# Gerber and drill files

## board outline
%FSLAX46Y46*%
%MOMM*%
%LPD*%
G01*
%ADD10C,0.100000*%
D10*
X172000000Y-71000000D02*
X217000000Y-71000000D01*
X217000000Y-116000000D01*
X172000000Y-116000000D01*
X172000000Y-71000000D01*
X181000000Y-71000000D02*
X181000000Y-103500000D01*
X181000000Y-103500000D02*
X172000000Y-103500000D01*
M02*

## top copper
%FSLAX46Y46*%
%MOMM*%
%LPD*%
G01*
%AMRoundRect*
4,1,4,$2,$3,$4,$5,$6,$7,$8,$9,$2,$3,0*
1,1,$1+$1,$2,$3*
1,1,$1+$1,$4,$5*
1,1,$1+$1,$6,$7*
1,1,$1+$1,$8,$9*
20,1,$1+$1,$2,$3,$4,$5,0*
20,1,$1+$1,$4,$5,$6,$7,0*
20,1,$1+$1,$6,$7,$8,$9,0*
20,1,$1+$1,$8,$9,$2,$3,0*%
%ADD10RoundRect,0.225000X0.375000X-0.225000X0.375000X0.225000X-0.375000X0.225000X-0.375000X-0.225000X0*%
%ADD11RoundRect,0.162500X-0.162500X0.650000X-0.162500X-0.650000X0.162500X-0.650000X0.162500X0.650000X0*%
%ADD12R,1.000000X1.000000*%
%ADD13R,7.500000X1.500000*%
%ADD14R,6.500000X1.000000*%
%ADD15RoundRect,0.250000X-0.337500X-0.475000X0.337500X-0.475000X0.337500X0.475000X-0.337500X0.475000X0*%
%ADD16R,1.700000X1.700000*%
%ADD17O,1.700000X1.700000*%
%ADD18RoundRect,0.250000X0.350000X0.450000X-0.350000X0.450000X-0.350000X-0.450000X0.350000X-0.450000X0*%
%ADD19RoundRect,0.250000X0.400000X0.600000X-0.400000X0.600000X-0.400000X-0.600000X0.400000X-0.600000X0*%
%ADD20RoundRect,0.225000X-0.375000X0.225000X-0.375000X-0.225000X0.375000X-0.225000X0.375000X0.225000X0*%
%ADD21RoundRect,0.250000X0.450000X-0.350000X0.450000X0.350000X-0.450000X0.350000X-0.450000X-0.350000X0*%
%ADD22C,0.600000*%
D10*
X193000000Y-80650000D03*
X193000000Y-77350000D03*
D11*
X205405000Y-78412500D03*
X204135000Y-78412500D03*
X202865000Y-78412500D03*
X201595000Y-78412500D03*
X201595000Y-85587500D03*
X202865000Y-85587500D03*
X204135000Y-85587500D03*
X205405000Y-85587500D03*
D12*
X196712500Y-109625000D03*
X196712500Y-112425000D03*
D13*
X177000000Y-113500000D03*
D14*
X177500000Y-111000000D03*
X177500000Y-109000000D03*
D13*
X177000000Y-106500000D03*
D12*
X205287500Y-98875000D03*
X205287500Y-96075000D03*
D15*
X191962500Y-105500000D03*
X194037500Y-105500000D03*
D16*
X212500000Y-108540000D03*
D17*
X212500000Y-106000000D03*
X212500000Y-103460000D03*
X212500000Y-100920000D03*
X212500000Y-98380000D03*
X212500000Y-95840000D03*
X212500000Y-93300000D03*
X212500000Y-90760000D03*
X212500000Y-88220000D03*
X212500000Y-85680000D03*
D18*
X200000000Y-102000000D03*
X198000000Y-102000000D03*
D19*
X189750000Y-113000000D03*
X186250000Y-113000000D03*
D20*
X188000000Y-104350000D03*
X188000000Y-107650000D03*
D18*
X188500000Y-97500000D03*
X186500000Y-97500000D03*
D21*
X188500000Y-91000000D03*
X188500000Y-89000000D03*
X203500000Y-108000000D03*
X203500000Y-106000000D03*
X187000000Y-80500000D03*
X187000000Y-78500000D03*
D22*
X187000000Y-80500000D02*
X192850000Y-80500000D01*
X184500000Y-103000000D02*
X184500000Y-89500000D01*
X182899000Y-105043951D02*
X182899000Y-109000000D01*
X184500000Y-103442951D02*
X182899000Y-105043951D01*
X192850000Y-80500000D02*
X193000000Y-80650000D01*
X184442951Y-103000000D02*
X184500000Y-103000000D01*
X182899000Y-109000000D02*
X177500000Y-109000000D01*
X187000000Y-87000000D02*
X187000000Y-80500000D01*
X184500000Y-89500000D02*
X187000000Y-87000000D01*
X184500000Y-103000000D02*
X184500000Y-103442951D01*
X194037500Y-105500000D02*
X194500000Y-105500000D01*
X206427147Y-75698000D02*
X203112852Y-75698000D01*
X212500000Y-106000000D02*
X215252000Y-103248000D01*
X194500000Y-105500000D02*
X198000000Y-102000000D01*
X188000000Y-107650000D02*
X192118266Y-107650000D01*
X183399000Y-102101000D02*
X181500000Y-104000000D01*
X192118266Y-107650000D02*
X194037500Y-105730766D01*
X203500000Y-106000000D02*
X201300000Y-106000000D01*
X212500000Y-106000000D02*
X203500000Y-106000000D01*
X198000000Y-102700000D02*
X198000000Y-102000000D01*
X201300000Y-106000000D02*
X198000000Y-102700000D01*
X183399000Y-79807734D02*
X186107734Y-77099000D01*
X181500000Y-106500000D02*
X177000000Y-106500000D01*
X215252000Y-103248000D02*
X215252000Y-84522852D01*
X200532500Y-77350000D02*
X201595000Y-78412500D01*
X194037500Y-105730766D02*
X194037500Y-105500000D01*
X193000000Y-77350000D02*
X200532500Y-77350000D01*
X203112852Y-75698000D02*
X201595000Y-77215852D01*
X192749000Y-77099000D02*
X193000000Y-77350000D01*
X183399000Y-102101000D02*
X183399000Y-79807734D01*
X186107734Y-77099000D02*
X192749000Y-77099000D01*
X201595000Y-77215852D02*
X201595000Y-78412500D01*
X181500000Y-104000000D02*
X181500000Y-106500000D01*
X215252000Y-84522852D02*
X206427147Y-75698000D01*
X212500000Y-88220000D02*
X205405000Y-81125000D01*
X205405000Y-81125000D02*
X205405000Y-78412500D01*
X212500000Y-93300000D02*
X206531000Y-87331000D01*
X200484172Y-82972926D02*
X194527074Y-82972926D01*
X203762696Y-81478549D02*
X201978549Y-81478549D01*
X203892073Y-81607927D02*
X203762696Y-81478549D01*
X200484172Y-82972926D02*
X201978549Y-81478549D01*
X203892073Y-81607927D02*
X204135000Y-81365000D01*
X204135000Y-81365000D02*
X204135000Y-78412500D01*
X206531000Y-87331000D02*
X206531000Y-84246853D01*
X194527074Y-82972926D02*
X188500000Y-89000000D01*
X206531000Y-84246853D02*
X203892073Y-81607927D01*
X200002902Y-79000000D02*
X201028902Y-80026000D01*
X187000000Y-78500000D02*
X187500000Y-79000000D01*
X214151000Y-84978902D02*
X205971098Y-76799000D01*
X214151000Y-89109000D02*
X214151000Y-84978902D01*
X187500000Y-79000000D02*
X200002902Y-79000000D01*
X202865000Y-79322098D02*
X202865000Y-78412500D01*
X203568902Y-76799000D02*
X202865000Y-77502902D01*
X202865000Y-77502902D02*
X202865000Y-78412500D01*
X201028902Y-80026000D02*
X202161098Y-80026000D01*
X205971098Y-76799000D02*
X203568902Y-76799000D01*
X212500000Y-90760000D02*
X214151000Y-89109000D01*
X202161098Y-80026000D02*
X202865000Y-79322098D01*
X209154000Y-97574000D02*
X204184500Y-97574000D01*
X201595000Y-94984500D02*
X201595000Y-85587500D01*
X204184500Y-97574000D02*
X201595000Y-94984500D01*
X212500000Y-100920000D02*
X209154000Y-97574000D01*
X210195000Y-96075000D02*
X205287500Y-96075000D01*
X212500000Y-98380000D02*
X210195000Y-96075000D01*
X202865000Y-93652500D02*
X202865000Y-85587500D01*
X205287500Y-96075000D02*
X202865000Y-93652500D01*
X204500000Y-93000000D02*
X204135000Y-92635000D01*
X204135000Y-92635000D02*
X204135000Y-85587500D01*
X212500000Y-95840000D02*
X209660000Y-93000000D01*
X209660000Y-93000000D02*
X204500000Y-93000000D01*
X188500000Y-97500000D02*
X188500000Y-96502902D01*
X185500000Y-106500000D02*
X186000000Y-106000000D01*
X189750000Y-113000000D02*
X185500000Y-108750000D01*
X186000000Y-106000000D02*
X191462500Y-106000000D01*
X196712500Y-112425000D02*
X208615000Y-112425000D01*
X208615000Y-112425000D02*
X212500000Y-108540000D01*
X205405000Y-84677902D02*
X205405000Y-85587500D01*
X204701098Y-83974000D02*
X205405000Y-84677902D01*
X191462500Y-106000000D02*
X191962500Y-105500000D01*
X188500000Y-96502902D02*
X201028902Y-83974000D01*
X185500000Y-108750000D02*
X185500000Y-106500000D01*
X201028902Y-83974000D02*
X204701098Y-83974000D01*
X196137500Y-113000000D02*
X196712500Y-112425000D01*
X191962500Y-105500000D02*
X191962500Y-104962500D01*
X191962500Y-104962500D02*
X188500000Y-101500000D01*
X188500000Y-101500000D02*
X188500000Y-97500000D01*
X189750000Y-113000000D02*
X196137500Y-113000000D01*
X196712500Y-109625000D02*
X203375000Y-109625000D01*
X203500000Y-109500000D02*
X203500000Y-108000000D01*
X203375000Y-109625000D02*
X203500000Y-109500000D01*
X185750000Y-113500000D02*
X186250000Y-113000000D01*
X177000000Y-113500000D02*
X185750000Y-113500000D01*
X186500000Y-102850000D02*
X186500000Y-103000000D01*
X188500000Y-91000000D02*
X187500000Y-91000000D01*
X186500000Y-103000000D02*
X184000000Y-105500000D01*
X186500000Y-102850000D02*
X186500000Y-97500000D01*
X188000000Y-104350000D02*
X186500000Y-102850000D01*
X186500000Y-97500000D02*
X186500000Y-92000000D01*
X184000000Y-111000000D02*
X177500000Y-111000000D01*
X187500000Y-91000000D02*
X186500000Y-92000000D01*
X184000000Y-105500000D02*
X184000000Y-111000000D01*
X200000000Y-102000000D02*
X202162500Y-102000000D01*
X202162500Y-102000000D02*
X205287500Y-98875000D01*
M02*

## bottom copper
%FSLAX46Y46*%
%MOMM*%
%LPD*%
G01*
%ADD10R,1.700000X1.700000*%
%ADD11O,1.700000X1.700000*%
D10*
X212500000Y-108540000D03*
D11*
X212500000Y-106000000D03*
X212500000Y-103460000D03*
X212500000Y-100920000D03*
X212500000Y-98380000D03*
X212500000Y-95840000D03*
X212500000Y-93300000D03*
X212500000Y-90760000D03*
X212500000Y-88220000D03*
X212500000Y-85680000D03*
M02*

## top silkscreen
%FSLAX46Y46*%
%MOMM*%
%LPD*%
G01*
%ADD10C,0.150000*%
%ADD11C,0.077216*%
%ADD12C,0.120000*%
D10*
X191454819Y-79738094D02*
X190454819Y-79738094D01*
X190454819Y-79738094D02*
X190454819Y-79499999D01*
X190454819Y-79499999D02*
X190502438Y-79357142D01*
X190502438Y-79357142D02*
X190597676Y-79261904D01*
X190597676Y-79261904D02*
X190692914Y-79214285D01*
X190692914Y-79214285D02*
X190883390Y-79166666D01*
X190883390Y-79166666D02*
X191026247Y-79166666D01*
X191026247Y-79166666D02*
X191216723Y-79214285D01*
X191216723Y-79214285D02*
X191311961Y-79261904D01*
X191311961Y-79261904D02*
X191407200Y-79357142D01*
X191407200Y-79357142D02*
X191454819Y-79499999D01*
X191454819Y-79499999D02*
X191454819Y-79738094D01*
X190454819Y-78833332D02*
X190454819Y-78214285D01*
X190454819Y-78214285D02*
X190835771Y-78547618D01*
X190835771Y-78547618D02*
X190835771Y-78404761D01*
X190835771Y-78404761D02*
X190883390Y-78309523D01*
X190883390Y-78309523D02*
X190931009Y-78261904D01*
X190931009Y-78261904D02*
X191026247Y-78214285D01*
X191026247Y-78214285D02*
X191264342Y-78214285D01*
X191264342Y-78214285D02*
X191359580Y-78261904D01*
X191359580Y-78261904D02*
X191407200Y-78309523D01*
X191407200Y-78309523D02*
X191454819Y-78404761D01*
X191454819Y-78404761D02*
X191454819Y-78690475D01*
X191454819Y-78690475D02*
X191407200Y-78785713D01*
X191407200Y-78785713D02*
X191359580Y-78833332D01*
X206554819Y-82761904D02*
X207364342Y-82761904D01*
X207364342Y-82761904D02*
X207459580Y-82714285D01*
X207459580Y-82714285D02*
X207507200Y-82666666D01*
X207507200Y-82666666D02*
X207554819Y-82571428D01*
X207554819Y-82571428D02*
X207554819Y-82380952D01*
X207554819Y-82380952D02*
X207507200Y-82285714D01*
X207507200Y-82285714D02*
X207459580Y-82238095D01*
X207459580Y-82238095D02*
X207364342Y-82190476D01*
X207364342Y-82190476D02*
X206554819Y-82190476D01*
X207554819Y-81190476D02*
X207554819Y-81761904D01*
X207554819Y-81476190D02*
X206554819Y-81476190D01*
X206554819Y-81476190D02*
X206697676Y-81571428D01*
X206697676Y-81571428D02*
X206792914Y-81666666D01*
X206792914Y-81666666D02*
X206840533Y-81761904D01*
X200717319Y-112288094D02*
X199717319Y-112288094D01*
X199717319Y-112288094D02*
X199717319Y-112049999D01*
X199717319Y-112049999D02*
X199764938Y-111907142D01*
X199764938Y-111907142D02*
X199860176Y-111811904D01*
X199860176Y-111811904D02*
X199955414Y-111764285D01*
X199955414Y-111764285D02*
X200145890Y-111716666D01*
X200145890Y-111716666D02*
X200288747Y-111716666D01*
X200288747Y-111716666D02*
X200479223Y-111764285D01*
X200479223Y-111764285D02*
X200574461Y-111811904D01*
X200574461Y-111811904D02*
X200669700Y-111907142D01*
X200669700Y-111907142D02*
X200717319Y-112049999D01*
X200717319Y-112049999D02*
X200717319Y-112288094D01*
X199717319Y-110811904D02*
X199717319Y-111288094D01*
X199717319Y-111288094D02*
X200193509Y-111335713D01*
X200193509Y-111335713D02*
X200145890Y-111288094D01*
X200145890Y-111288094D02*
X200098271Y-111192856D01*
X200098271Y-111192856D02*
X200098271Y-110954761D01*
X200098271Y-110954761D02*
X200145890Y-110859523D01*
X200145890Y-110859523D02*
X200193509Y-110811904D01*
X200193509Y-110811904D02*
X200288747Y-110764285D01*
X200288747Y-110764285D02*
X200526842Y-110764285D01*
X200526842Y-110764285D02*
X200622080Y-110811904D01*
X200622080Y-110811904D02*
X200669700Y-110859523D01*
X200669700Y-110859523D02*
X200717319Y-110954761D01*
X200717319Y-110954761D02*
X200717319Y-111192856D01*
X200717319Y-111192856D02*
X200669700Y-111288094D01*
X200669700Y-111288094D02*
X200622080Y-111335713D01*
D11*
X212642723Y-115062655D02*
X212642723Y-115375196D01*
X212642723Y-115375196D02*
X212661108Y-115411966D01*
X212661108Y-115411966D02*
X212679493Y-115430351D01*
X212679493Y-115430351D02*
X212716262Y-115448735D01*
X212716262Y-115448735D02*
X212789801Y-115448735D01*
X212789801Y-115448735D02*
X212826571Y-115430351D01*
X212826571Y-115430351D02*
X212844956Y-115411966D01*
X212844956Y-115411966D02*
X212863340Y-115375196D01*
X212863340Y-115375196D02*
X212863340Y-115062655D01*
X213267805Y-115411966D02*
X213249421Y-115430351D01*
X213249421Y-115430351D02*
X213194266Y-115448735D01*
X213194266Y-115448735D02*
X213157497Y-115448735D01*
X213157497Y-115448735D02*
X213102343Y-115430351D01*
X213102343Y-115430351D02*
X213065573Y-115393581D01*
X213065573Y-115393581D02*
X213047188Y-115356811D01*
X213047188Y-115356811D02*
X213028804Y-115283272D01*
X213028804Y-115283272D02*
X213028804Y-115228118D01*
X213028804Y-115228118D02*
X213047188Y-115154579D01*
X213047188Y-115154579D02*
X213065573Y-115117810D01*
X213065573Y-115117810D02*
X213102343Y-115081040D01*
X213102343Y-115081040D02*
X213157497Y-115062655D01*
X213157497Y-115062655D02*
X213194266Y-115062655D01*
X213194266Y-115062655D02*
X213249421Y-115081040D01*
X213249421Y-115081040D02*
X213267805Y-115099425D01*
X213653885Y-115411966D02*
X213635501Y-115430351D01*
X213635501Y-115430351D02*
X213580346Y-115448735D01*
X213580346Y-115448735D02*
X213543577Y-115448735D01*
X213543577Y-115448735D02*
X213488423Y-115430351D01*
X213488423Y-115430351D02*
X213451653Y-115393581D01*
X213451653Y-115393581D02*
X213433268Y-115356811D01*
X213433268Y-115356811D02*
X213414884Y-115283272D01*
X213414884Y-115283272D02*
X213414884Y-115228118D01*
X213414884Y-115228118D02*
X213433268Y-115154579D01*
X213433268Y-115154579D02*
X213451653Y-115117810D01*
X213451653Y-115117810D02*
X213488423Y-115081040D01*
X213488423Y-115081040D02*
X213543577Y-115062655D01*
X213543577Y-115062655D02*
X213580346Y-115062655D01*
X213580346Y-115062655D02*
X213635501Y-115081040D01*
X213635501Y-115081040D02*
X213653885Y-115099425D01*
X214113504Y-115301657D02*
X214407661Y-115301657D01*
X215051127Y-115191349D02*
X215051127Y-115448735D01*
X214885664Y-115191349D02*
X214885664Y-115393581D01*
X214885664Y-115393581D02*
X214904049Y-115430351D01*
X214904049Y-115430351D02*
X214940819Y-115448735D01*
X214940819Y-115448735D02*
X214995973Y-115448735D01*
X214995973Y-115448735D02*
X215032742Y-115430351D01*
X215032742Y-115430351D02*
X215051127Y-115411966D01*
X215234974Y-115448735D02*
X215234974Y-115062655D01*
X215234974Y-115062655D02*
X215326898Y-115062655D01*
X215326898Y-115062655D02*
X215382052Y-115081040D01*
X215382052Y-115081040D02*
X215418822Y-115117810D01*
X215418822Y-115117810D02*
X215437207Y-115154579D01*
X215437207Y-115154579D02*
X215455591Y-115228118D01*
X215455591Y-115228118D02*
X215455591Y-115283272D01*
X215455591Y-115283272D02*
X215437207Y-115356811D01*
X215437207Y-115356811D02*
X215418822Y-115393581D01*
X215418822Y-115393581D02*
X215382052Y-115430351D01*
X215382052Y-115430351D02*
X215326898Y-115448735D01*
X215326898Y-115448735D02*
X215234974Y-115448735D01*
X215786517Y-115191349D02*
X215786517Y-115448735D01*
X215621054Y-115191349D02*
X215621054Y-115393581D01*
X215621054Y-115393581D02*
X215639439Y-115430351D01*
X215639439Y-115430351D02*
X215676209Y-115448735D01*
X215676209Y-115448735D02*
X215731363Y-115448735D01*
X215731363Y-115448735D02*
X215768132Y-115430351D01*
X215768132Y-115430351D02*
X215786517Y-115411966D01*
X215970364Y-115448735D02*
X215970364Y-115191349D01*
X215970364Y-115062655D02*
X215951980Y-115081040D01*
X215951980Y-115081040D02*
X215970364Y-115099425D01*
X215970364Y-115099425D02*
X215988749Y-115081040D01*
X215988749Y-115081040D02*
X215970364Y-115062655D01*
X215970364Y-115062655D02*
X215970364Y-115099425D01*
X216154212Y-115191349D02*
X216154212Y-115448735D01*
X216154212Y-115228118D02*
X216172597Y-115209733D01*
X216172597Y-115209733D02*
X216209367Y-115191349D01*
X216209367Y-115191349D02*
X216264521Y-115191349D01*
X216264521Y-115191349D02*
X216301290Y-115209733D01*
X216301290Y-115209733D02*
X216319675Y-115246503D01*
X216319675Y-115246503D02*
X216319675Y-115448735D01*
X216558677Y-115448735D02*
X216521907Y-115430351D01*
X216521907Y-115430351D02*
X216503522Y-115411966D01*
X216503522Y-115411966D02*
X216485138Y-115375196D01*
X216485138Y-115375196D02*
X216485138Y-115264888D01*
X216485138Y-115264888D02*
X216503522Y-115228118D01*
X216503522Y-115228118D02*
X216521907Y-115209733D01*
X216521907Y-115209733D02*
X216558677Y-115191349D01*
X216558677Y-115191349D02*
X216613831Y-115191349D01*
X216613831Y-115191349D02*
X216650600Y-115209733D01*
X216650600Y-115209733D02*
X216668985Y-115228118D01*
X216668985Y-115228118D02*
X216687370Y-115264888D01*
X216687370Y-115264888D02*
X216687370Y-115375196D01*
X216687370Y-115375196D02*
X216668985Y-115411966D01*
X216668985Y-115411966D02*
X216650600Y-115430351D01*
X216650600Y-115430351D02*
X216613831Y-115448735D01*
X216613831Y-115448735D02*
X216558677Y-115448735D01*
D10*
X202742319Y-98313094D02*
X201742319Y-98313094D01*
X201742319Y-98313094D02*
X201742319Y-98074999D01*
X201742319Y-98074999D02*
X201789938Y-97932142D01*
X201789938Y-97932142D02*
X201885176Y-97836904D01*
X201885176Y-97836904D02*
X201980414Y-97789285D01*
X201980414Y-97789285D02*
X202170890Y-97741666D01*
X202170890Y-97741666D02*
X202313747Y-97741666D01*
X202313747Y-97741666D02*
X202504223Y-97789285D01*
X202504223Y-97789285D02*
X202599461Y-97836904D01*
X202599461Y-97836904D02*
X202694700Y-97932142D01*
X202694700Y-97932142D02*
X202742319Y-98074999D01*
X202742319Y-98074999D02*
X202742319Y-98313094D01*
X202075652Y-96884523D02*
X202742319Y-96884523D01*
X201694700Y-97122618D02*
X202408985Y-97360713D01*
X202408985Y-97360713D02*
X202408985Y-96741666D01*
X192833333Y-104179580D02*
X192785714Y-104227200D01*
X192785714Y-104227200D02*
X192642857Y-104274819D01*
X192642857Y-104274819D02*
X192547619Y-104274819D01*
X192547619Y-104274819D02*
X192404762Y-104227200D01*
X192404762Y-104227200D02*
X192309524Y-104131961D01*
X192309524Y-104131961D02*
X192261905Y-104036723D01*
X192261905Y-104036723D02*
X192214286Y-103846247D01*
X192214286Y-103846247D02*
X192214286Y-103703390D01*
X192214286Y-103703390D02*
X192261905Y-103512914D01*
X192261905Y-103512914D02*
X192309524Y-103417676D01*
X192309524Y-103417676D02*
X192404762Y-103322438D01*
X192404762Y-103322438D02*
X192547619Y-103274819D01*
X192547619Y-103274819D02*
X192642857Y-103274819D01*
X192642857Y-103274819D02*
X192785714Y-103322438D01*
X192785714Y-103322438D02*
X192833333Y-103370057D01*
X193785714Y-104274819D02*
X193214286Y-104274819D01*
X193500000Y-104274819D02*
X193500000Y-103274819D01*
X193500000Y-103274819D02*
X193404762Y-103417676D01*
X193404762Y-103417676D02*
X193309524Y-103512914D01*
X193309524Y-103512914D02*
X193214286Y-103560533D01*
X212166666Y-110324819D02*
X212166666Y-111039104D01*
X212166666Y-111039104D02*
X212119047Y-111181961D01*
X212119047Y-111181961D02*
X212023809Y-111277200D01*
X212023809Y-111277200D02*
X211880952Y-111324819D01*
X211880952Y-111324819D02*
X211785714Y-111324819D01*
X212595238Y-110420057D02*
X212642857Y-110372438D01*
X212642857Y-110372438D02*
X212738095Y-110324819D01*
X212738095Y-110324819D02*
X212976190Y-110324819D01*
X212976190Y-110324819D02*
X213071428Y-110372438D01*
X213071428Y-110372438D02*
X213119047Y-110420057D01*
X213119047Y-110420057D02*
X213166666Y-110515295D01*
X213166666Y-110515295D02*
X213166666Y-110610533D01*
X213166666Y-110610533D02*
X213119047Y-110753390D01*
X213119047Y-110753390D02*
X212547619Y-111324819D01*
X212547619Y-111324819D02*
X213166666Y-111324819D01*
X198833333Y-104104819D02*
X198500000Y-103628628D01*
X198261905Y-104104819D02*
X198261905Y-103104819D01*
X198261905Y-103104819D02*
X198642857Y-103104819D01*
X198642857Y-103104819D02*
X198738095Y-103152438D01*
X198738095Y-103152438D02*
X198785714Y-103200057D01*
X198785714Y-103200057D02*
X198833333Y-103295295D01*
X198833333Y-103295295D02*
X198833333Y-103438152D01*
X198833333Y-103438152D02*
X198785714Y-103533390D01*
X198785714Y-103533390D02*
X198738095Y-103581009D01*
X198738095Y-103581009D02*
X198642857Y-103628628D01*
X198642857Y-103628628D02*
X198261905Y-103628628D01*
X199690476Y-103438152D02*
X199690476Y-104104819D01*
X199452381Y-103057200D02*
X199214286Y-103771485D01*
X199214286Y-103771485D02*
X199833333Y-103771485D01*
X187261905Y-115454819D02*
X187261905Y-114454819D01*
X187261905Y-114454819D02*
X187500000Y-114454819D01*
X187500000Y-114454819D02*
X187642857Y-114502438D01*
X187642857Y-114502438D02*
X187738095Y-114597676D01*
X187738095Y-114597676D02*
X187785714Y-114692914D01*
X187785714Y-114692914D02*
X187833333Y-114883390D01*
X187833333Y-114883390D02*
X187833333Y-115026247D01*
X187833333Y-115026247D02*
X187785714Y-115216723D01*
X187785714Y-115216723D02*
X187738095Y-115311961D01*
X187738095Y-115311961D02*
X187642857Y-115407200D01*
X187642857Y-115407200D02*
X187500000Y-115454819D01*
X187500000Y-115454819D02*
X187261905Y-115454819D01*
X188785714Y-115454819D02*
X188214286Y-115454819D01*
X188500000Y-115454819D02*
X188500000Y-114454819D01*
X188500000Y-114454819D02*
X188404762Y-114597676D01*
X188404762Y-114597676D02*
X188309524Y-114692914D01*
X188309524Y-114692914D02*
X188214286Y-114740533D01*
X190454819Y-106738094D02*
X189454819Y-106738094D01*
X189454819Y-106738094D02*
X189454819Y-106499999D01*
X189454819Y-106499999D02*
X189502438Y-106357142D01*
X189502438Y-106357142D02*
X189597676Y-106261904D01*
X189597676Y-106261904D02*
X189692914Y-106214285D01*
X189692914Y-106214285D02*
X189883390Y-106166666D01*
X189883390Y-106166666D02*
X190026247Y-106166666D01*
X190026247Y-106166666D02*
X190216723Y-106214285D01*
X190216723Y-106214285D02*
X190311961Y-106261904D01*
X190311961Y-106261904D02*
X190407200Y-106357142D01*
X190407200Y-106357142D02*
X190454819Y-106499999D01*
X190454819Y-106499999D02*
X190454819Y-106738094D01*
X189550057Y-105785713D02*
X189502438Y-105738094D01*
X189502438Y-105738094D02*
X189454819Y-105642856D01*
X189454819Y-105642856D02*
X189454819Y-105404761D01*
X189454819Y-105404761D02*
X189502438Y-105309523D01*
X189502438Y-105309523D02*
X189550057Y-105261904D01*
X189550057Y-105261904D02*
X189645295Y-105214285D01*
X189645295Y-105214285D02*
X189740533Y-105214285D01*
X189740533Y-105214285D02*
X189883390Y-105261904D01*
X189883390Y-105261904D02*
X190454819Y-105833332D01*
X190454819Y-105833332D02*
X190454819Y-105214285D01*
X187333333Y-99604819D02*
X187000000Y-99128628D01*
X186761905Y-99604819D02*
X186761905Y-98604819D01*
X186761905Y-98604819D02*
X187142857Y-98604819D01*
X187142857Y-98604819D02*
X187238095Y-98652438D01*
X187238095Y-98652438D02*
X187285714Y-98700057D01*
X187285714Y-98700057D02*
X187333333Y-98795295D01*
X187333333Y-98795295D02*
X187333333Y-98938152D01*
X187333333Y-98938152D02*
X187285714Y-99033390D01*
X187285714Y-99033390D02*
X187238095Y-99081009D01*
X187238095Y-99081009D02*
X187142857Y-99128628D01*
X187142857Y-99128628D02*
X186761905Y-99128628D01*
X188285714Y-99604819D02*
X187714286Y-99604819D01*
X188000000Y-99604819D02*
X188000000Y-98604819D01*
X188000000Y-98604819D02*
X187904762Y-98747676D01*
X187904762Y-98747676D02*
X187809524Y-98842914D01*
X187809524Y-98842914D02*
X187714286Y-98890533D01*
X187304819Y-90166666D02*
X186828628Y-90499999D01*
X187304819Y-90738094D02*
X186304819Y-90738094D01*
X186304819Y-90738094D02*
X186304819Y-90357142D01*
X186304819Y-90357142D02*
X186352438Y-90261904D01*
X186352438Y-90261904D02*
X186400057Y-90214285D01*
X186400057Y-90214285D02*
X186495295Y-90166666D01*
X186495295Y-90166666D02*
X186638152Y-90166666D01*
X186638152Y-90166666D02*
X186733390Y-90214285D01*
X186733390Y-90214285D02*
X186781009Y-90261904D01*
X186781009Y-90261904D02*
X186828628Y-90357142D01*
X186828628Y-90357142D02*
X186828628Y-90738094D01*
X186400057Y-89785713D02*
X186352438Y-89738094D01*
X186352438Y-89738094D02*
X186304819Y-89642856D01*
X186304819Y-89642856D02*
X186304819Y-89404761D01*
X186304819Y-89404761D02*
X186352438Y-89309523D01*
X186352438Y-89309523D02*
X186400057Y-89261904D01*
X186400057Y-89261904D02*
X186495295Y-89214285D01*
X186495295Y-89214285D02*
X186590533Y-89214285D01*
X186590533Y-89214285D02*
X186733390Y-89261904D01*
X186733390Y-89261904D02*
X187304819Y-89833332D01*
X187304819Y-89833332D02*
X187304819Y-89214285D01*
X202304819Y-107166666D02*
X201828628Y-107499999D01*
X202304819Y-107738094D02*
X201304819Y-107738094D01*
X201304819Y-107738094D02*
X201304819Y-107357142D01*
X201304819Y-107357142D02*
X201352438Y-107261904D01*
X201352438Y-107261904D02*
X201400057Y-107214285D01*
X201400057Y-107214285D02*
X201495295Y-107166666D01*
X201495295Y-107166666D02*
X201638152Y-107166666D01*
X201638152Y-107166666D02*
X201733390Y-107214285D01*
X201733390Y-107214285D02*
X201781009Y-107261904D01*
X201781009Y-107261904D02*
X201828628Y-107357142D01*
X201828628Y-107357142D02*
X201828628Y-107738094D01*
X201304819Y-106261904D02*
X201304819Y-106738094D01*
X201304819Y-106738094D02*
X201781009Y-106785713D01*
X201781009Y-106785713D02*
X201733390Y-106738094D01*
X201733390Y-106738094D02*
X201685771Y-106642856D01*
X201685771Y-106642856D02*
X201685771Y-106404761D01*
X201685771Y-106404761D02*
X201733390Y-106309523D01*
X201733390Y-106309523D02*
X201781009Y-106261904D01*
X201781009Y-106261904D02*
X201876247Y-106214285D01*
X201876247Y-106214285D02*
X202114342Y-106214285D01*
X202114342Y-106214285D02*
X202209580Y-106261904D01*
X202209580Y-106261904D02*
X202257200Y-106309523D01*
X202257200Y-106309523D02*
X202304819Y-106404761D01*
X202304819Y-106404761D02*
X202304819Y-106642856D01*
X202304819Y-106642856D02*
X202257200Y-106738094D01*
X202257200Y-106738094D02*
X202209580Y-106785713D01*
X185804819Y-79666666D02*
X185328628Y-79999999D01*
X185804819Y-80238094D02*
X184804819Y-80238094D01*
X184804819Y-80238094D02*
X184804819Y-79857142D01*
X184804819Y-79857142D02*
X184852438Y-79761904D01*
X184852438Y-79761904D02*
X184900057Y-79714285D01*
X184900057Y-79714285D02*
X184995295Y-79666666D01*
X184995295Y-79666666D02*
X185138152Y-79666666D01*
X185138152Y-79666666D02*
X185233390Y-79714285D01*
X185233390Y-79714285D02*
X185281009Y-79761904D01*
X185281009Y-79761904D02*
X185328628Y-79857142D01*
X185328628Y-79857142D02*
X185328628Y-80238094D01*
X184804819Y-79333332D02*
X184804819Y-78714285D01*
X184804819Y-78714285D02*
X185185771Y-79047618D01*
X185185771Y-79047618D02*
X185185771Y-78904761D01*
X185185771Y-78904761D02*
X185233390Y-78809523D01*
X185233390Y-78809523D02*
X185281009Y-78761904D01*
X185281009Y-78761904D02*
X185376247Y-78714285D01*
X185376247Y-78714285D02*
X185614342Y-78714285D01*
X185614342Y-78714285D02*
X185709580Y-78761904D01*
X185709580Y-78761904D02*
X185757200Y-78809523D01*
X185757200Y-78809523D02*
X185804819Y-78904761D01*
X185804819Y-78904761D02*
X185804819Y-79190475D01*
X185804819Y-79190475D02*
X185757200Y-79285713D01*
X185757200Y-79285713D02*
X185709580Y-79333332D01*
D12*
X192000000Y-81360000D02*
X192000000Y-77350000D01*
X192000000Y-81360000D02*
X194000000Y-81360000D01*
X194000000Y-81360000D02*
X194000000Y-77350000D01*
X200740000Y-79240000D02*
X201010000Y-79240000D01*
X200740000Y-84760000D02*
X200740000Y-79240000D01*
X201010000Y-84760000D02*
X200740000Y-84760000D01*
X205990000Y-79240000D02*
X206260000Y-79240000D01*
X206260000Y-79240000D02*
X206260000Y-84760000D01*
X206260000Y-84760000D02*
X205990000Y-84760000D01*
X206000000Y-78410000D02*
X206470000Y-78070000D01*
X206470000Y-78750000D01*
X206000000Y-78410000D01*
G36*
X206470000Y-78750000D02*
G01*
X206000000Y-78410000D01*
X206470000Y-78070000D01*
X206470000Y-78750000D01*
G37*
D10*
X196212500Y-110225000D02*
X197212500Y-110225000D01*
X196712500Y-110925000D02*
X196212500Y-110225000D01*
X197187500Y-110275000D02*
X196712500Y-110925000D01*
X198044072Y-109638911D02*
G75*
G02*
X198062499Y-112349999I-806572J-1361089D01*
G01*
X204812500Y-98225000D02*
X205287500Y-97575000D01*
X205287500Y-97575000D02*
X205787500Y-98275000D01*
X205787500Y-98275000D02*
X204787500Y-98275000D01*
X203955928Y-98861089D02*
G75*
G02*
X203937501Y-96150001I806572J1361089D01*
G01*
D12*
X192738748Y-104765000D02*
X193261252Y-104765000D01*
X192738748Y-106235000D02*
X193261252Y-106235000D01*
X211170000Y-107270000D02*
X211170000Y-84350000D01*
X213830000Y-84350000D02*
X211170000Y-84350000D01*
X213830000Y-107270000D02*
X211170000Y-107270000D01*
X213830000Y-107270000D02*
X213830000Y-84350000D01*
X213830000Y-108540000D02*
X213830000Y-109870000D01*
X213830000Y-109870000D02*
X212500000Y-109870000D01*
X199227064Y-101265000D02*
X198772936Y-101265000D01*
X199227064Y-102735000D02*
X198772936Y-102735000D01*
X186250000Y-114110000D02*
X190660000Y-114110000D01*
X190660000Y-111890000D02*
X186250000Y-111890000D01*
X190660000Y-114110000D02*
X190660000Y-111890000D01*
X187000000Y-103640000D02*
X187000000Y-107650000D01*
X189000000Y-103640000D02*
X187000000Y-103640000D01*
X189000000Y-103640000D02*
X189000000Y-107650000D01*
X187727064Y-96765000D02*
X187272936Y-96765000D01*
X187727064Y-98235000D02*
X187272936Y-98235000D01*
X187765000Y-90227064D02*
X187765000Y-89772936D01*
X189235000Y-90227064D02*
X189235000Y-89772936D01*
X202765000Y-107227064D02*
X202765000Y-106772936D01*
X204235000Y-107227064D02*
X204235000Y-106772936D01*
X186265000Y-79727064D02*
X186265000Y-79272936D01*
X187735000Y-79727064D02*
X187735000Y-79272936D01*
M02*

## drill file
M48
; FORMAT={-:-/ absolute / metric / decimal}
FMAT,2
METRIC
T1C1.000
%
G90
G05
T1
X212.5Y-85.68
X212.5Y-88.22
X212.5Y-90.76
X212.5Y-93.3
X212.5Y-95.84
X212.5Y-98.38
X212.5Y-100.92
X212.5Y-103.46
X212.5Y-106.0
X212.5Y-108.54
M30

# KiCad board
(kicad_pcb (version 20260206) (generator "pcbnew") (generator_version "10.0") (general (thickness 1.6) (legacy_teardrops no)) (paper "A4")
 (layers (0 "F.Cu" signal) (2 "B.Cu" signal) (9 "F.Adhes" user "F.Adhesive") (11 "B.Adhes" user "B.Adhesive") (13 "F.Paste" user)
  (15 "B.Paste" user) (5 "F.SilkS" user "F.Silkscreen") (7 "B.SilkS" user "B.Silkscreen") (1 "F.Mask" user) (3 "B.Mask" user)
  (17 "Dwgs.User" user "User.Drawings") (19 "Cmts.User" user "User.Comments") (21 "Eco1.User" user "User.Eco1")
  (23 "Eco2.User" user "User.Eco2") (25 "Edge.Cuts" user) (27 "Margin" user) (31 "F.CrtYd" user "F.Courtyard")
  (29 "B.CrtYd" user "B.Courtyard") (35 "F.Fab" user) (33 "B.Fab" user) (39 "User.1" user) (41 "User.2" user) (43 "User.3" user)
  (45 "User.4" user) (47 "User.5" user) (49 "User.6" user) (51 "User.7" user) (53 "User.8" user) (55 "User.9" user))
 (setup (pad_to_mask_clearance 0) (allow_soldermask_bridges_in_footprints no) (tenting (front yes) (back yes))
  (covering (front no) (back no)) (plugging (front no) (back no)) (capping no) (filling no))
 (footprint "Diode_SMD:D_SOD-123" (layer "F.Cu") (at 193 79 90)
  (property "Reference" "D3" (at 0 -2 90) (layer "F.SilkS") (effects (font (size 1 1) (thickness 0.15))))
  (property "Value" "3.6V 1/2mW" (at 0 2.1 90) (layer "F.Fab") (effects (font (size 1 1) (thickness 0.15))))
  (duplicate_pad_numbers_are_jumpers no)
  (fp_line (start -2.36 -1) (end 1.65 -1) (stroke (width 0.12) (type solid)) (layer "F.SilkS"))
  (fp_line (start -2.36 -1) (end -2.36 1) (stroke (width 0.12) (type solid)) (layer "F.SilkS"))
  (fp_line (start -2.36 1) (end 1.65 1) (stroke (width 0.12) (type solid)) (layer "F.SilkS"))
  (pad "1" smd roundrect (at -1.65 0 90) (size 0.9 1.2) (layers "F.Cu" "F.Mask" "F.Paste") (roundrect_rratio 0.25) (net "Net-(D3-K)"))
  (pad "2" smd roundrect (at 1.65 0 90) (size 0.9 1.2) (layers "F.Cu" "F.Mask" "F.Paste") (roundrect_rratio 0.25) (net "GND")))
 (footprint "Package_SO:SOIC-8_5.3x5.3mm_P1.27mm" (layer "F.Cu") (at 203.5 82 -90)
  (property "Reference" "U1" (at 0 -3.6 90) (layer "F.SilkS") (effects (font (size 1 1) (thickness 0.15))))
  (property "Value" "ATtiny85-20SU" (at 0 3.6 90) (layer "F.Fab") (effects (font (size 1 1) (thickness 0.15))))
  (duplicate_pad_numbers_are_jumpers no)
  (fp_line (start -2.76 2.76) (end -2.76 2.49) (stroke (width 0.12) (type solid)) (layer "F.SilkS"))
  (fp_line (start 2.76 2.76) (end -2.76 2.76) (stroke (width 0.12) (type solid)) (layer "F.SilkS"))
  (fp_line (start 2.76 2.49) (end 2.76 2.76) (stroke (width 0.12) (type solid)) (layer "F.SilkS"))
  (fp_line (start -2.76 -2.49) (end -2.76 -2.76) (stroke (width 0.12) (type solid)) (layer "F.SilkS"))
  (fp_line (start -2.76 -2.76) (end 2.76 -2.76) (stroke (width 0.12) (type solid)) (layer "F.SilkS"))
  (fp_line (start 2.76 -2.76) (end 2.76 -2.49) (stroke (width 0.12) (type solid)) (layer "F.SilkS"))
  (fp_poly (pts (xy -3.59 -2.5) (xy -3.93 -2.97) (xy -3.25 -2.97)) (stroke (width 0.12) (type solid)) (fill yes) (layer "F.SilkS"))
  (pad "1" smd roundrect (at -3.5875 -1.905 270) (size 1.625 0.65) (layers "F.Cu" "F.Mask" "F.Paste") (roundrect_rratio 0.25)
   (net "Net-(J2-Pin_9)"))
  (pad "2" smd roundrect (at -3.5875 -0.635 270) (size 1.625 0.65) (layers "F.Cu" "F.Mask" "F.Paste") (roundrect_rratio 0.25)
   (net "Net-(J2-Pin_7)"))
  (pad "3" smd roundrect (at -3.5875 0.635 270) (size 1.625 0.65) (layers "F.Cu" "F.Mask" "F.Paste") (roundrect_rratio 0.25)
   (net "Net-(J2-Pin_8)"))
  (pad "4" smd roundrect (at -3.5875 1.905 270) (size 1.625 0.65) (layers "F.Cu" "F.Mask" "F.Paste") (roundrect_rratio 0.25) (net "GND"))
  (pad "5" smd roundrect (at 3.5875 1.905 270) (size 1.625 0.65) (layers "F.Cu" "F.Mask" "F.Paste") (roundrect_rratio 0.25)
   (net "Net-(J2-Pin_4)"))
  (pad "6" smd roundrect (at 3.5875 0.635 270) (size 1.625 0.65) (layers "F.Cu" "F.Mask" "F.Paste") (roundrect_rratio 0.25)
   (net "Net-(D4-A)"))
  (pad "7" smd roundrect (at 3.5875 -0.635 270) (size 1.625 0.65) (layers "F.Cu" "F.Mask" "F.Paste") (roundrect_rratio 0.25)
   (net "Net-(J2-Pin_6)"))
  (pad "8" smd roundrect (at 3.5875 -1.905 270) (size 1.625 0.65) (layers "F.Cu" "F.Mask" "F.Paste") (roundrect_rratio 0.25) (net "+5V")))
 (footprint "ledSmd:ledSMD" (layer "F.Cu") (at 196.7125 111.425 -90)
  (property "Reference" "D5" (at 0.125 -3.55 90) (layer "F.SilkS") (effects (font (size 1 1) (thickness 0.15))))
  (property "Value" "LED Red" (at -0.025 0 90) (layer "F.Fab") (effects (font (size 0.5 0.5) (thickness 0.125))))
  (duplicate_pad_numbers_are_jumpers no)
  (fp_line (start -1.2 0.5) (end -1.2 -0.5) (stroke (width 0.15) (type solid)) (layer "F.SilkS"))
  (fp_line (start -0.5 0) (end -1.2 0.5) (stroke (width 0.15) (type solid)) (layer "F.SilkS"))
  (fp_line (start -1.15 -0.475) (end -0.5 0) (stroke (width 0.15) (type solid)) (layer "F.SilkS"))
  (fp_arc (start -1.786089 -1.331572) (mid -0.435753 -2.107089) (end 0.924999 -1.349999) (stroke (width 0.15) (type solid))
   (layer "F.SilkS"))
  (pad "1" smd rect (at -1.8 0 270) (size 1 1) (layers "F.Cu" "F.Mask" "F.Paste") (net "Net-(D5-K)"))
  (pad "2" smd rect (at 1 0 270) (size 1 1) (layers "F.Cu" "F.Mask" "F.Paste") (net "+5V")))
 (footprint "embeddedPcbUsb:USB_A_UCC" (layer "F.Cu") (at 177.2 110)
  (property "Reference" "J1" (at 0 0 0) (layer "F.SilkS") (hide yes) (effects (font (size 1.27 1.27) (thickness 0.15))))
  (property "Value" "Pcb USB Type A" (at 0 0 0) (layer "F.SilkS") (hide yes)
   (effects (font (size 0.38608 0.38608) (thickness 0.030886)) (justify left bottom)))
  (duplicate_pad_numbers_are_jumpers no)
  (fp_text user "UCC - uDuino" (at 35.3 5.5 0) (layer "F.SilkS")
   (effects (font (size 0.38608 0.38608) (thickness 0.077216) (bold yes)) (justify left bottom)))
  (pad "1" smd rect (at -0.2 3.5) (size 7.5 1.5) (layers "F.Cu" "F.Mask" "F.Paste") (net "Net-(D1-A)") (solder_mask_margin 0.1016))
  (pad "2" smd rect (at 0.3 1) (size 6.5 1) (layers "F.Cu" "F.Mask" "F.Paste") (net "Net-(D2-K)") (solder_mask_margin 0.1016))
  (pad "3" smd rect (at 0.3 -1) (size 6.5 1) (layers "F.Cu" "F.Mask" "F.Paste") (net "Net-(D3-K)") (solder_mask_margin 0.1016))
  (pad "4" smd rect (at -0.2 -3.5) (size 7.5 1.5) (layers "F.Cu" "F.Mask" "F.Paste") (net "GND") (solder_mask_margin 0.1016)))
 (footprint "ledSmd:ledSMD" (layer "F.Cu") (at 205.2875 97.075 90)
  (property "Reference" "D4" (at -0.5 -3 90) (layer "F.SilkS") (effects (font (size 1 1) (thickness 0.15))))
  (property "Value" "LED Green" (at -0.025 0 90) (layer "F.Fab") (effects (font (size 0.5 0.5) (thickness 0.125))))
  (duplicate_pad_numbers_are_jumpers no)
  (fp_line (start -1.15 -0.475) (end -0.5 0) (stroke (width 0.15) (type solid)) (layer "F.SilkS"))
  (fp_line (start -0.5 0) (end -1.2 0.5) (stroke (width 0.15) (type solid)) (layer "F.SilkS"))
  (fp_line (start -1.2 0.5) (end -1.2 -0.5) (stroke (width 0.15) (type solid)) (layer "F.SilkS"))
  (fp_arc (start -1.786089 -1.331572) (mid -0.435753 -2.107089) (end 0.924999 -1.349999) (stroke (width 0.15) (type solid))
   (layer "F.SilkS"))
  (pad "1" smd rect (at -1.8 0 90) (size 1 1) (layers "F.Cu" "F.Mask" "F.Paste") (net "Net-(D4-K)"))
  (pad "2" smd rect (at 1 0 90) (size 1 1) (layers "F.Cu" "F.Mask" "F.Paste") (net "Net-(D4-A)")))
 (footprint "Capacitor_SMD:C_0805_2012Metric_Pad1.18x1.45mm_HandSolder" (layer "F.Cu") (at 193 105.5)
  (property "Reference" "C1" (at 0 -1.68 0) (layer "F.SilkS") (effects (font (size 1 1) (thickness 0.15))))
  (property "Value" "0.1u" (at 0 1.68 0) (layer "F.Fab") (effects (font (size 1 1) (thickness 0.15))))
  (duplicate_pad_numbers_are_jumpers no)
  (fp_line (start -0.261252 -0.735) (end 0.261252 -0.735) (stroke (width 0.12) (type solid)) (layer "F.SilkS"))
  (fp_line (start -0.261252 0.735) (end 0.261252 0.735) (stroke (width 0.12) (type solid)) (layer "F.SilkS"))
  (pad "1" smd roundrect (at -1.0375 0) (size 1.175 1.45) (layers "F.Cu" "F.Mask" "F.Paste") (roundrect_rratio 0.212766) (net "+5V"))
  (pad "2" smd roundrect (at 1.0375 0) (size 1.175 1.45) (layers "F.Cu" "F.Mask" "F.Paste") (roundrect_rratio 0.212766) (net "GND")))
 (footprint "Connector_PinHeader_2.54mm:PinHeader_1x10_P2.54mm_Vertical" (layer "F.Cu") (at 212.5 108.54 180)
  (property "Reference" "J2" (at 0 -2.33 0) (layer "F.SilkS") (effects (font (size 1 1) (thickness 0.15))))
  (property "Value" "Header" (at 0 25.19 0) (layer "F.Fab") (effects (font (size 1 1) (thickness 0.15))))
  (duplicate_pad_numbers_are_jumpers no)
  (fp_line (start 1.33 1.27) (end 1.33 24.19) (stroke (width 0.12) (type solid)) (layer "F.SilkS"))
  (fp_line (start -1.33 24.19) (end 1.33 24.19) (stroke (width 0.12) (type solid)) (layer "F.SilkS"))
  (fp_line (start -1.33 1.27) (end 1.33 1.27) (stroke (width 0.12) (type solid)) (layer "F.SilkS"))
  (fp_line (start -1.33 1.27) (end -1.33 24.19) (stroke (width 0.12) (type solid)) (layer "F.SilkS"))
  (fp_line (start -1.33 0) (end -1.33 -1.33) (stroke (width 0.12) (type solid)) (layer "F.SilkS"))
  (fp_line (start -1.33 -1.33) (end 0 -1.33) (stroke (width 0.12) (type solid)) (layer "F.SilkS"))
  (pad "1" thru_hole rect (at 0 0 180) (size 1.7 1.7) (drill 1) (layers "*.Cu" "*.Mask") (remove_unused_layers no) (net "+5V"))
  (pad "2" thru_hole oval (at 0 2.54 180) (size 1.7 1.7) (drill 1) (layers "*.Cu" "*.Mask") (remove_unused_layers no) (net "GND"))
  (pad "3" thru_hole oval (at 0 5.08 180) (size 1.7 1.7) (drill 1) (layers "*.Cu" "*.Mask") (remove_unused_layers no)
   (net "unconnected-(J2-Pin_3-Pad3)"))
  (pad "4" thru_hole oval (at 0 7.62 180) (size 1.7 1.7) (drill 1) (layers "*.Cu" "*.Mask") (remove_unused_layers no) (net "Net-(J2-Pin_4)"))
  (pad "5" thru_hole oval (at 0 10.16 180) (size 1.7 1.7) (drill 1) (layers "*.Cu" "*.Mask") (remove_unused_layers no) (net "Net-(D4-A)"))
  (pad "6" thru_hole oval (at 0 12.7 180) (size 1.7 1.7) (drill 1) (layers "*.Cu" "*.Mask") (remove_unused_layers no) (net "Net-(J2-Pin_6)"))
  (pad "7" thru_hole oval (at 0 15.24 180) (size 1.7 1.7) (drill 1) (layers "*.Cu" "*.Mask") (remove_unused_layers no)
   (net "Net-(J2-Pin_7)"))
  (pad "8" thru_hole oval (at 0 17.78 180) (size 1.7 1.7) (drill 1) (layers "*.Cu" "*.Mask") (remove_unused_layers no)
   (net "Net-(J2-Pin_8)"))
  (pad "9" thru_hole oval (at 0 20.32 180) (size 1.7 1.7) (drill 1) (layers "*.Cu" "*.Mask") (remove_unused_layers no)
   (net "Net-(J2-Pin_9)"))
  (pad "10" thru_hole oval (at 0 22.86 180) (size 1.7 1.7) (drill 1) (layers "*.Cu" "*.Mask") (remove_unused_layers no)
   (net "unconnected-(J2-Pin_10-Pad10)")))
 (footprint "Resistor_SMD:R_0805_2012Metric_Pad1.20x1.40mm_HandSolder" (layer "F.Cu") (at 199 102 180)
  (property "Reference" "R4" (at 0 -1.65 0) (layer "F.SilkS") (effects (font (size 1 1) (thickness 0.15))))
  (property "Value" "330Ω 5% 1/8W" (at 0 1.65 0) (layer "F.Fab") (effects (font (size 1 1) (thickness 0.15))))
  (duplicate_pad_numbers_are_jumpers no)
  (fp_line (start -0.227064 0.735) (end 0.227064 0.735) (stroke (width 0.12) (type solid)) (layer "F.SilkS"))
  (fp_line (start -0.227064 -0.735) (end 0.227064 -0.735) (stroke (width 0.12) (type solid)) (layer "F.SilkS"))
  (pad "1" smd roundrect (at -1 0 180) (size 1.2 1.4) (layers "F.Cu" "F.Mask" "F.Paste") (roundrect_rratio 0.208333) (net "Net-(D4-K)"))
  (pad "2" smd roundrect (at 1 0 180) (size 1.2 1.4) (layers "F.Cu" "F.Mask" "F.Paste") (roundrect_rratio 0.208333) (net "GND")))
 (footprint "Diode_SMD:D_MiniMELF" (layer "F.Cu") (at 188 113 180)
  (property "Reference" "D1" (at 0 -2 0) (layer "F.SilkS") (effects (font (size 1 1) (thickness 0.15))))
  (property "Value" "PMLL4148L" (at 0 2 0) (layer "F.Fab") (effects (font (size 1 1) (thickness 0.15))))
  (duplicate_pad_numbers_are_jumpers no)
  (fp_line (start 1.75 -1.11) (end -2.66 -1.11) (stroke (width 0.12) (type solid)) (layer "F.SilkS"))
  (fp_line (start -2.66 1.11) (end 1.75 1.11) (stroke (width 0.12) (type solid)) (layer "F.SilkS"))
  (fp_line (start -2.66 -1.11) (end -2.66 1.11) (stroke (width 0.12) (type solid)) (layer "F.SilkS"))
  (pad "1" smd roundrect (at -1.75 0 180) (size 1.3 1.7) (layers "F.Cu" "F.Mask" "F.Paste") (roundrect_rratio 0.1923076923) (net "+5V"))
  (pad "2" smd roundrect (at 1.75 0 180) (size 1.3 1.7) (layers "F.Cu" "F.Mask" "F.Paste") (roundrect_rratio 0.1923076923)
   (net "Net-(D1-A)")))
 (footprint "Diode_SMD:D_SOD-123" (layer "F.Cu") (at 188 106 -90)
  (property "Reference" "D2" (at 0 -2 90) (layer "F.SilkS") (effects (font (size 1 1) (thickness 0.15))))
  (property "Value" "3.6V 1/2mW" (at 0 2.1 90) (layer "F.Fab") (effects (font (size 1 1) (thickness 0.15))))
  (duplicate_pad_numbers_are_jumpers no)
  (fp_line (start -2.36 1) (end 1.65 1) (stroke (width 0.12) (type solid)) (layer "F.SilkS"))
  (fp_line (start -2.36 -1) (end -2.36 1) (stroke (width 0.12) (type solid)) (layer "F.SilkS"))
  (fp_line (start -2.36 -1) (end 1.65 -1) (stroke (width 0.12) (type solid)) (layer "F.SilkS"))
  (pad "1" smd roundrect (at -1.65 0 270) (size 0.9 1.2) (layers "F.Cu" "F.Mask" "F.Paste") (roundrect_rratio 0.25) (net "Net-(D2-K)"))
  (pad "2" smd roundrect (at 1.65 0 270) (size 0.9 1.2) (layers "F.Cu" "F.Mask" "F.Paste") (roundrect_rratio 0.25) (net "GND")))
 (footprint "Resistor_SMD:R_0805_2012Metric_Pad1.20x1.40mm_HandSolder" (layer "F.Cu") (at 187.5 97.5 180)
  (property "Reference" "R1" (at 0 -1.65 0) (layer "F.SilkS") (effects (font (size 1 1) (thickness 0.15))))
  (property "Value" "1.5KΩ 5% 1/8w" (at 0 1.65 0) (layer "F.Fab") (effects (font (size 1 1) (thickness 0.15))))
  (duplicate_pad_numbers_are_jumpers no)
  (fp_line (start -0.227064 0.735) (end 0.227064 0.735) (stroke (width 0.12) (type solid)) (layer "F.SilkS"))
  (fp_line (start -0.227064 -0.735) (end 0.227064 -0.735) (stroke (width 0.12) (type solid)) (layer "F.SilkS"))
  (pad "1" smd roundrect (at -1 0 180) (size 1.2 1.4) (layers "F.Cu" "F.Mask" "F.Paste") (roundrect_rratio 0.208333) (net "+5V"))
  (pad "2" smd roundrect (at 1 0 180) (size 1.2 1.4) (layers "F.Cu" "F.Mask" "F.Paste") (roundrect_rratio 0.208333) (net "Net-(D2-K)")))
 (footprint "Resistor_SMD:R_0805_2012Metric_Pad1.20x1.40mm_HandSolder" (layer "F.Cu") (at 188.5 90 90)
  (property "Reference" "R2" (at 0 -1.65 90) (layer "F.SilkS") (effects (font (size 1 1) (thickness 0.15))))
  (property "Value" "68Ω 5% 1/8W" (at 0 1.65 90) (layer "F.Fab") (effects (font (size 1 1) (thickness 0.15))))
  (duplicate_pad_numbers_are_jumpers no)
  (fp_line (start -0.227064 -0.735) (end 0.227064 -0.735) (stroke (width 0.12) (type solid)) (layer "F.SilkS"))
  (fp_line (start -0.227064 0.735) (end 0.227064 0.735) (stroke (width 0.12) (type solid)) (layer "F.SilkS"))
  (pad "1" smd roundrect (at -1 0 90) (size 1.2 1.4) (layers "F.Cu" "F.Mask" "F.Paste") (roundrect_rratio 0.208333) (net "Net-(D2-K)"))
  (pad "2" smd roundrect (at 1 0 90) (size 1.2 1.4) (layers "F.Cu" "F.Mask" "F.Paste") (roundrect_rratio 0.208333) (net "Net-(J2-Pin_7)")))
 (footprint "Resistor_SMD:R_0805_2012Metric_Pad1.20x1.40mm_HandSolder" (layer "F.Cu") (at 203.5 107 90)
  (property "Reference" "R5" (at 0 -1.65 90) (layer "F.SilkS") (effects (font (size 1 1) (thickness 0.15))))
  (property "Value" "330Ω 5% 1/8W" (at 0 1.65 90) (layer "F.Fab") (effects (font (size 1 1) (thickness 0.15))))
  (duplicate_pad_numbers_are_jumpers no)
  (fp_line (start -0.227064 -0.735) (end 0.227064 -0.735) (stroke (width 0.12) (type solid)) (layer "F.SilkS"))
  (fp_line (start -0.227064 0.735) (end 0.227064 0.735) (stroke (width 0.12) (type solid)) (layer "F.SilkS"))
  (pad "1" smd roundrect (at -1 0 90) (size 1.2 1.4) (layers "F.Cu" "F.Mask" "F.Paste") (roundrect_rratio 0.208333) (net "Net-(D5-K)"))
  (pad "2" smd roundrect (at 1 0 90) (size 1.2 1.4) (layers "F.Cu" "F.Mask" "F.Paste") (roundrect_rratio 0.208333) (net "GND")))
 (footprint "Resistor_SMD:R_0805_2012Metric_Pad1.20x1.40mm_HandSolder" (layer "F.Cu") (at 187 79.5 90)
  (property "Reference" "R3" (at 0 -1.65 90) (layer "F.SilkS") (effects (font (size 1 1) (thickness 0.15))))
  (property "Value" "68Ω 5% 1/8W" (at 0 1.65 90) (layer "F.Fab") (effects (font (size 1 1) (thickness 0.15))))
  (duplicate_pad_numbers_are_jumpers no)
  (fp_line (start -0.227064 -0.735) (end 0.227064 -0.735) (stroke (width 0.12) (type solid)) (layer "F.SilkS"))
  (fp_line (start -0.227064 0.735) (end 0.227064 0.735) (stroke (width 0.12) (type solid)) (layer "F.SilkS"))
  (pad "1" smd roundrect (at -1 0 90) (size 1.2 1.4) (layers "F.Cu" "F.Mask" "F.Paste") (roundrect_rratio 0.208333) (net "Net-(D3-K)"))
  (pad "2" smd roundrect (at 1 0 90) (size 1.2 1.4) (layers "F.Cu" "F.Mask" "F.Paste") (roundrect_rratio 0.208333) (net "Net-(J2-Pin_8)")))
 (gr_rect (start 172 71) (end 217 116) (stroke (width 0.1) (type default)) (fill no) (layer "Edge.Cuts"))
 (gr_line (start 181 71) (end 181 103.5) (stroke (width 0.1) (type default)) (layer "Edge.Cuts"))
 (gr_line (start 181 103.5) (end 172 103.5) (stroke (width 0.1) (type default)) (layer "Edge.Cuts"))
 (segment (start 187 80.5) (end 192.85 80.5) (width 0.6) (layer "F.Cu") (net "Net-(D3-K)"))
 (segment (start 184.5 103) (end 184.5 89.5) (width 0.6) (layer "F.Cu") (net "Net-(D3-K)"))
 (segment (start 182.899 105.043951) (end 182.899 109) (width 0.6) (layer "F.Cu") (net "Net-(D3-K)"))
 (segment (start 184.5 103.442951) (end 182.899 105.043951) (width 0.6) (layer "F.Cu") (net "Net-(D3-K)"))
 (segment (start 192.85 80.5) (end 193 80.65) (width 0.6) (layer "F.Cu") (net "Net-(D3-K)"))
 (segment (start 184.442951 103) (end 184.5 103) (width 0.6) (layer "F.Cu") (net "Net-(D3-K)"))
 (segment (start 182.899 109) (end 177.5 109) (width 0.6) (layer "F.Cu") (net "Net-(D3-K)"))
 (segment (start 187 87) (end 187 80.5) (width 0.6) (layer "F.Cu") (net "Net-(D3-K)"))
 (segment (start 184.5 89.5) (end 187 87) (width 0.6) (layer "F.Cu") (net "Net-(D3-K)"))
 (segment (start 184.5 103) (end 184.5 103.442951) (width 0.6) (layer "F.Cu") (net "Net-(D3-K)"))
 (segment (start 194.0375 105.5) (end 194.5 105.5) (width 0.6) (layer "F.Cu") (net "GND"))
 (segment (start 206.427147 75.698) (end 203.112852 75.698) (width 0.6) (layer "F.Cu") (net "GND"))
 (segment (start 212.5 106) (end 215.252 103.248) (width 0.6) (layer "F.Cu") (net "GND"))
 (segment (start 194.5 105.5) (end 198 102) (width 0.6) (layer "F.Cu") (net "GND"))
 (segment (start 188 107.65) (end 192.118266 107.65) (width 0.6) (layer "F.Cu") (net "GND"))
 (segment (start 183.399 102.101) (end 181.5 104) (width 0.6) (layer "F.Cu") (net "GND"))
 (segment (start 192.118266 107.65) (end 194.0375 105.730766) (width 0.6) (layer "F.Cu") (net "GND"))
 (segment (start 203.5 106) (end 201.3 106) (width 0.6) (layer "F.Cu") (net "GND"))
 (segment (start 212.5 106) (end 203.5 106) (width 0.6) (layer "F.Cu") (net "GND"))
 (segment (start 198 102.7) (end 198 102) (width 0.6) (layer "F.Cu") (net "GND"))
 (segment (start 201.3 106) (end 198 102.7) (width 0.6) (layer "F.Cu") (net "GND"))
 (segment (start 183.399 79.807734) (end 186.107734 77.099) (width 0.6) (layer "F.Cu") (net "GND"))
 (segment (start 181.5 106.5) (end 177 106.5) (width 0.6) (layer "F.Cu") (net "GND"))
 (segment (start 215.252 103.248) (end 215.252 84.522852) (width 0.6) (layer "F.Cu") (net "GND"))
 (segment (start 200.5325 77.35) (end 201.595 78.4125) (width 0.6) (layer "F.Cu") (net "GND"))
 (segment (start 194.0375 105.730766) (end 194.0375 105.5) (width 0.6) (layer "F.Cu") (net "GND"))
 (segment (start 193 77.35) (end 200.5325 77.35) (width 0.6) (layer "F.Cu") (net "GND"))
 (segment (start 203.112852 75.698) (end 201.595 77.215852) (width 0.6) (layer "F.Cu") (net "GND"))
 (segment (start 192.749 77.099) (end 193 77.35) (width 0.6) (layer "F.Cu") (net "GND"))
 (segment (start 183.399 102.101) (end 183.399 79.807734) (width 0.6) (layer "F.Cu") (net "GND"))
 (segment (start 186.107734 77.099) (end 192.749 77.099) (width 0.6) (layer "F.Cu") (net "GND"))
 (segment (start 201.595 77.215852) (end 201.595 78.4125) (width 0.6) (layer "F.Cu") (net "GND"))
 (segment (start 181.5 104) (end 181.5 106.5) (width 0.6) (layer "F.Cu") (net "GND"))
 (segment (start 215.252 84.522852) (end 206.427147 75.698) (width 0.6) (layer "F.Cu") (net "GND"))
 (segment (start 212.5 88.22) (end 205.405 81.125) (width 0.6) (layer "F.Cu") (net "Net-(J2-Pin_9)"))
 (segment (start 205.405 81.125) (end 205.405 78.4125) (width 0.6) (layer "F.Cu") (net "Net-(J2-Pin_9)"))
 (segment (start 212.5 93.3) (end 206.531 87.331) (width 0.6) (layer "F.Cu") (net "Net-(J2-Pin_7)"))
 (segment (start 200.484172 82.972926) (end 194.527074 82.972926) (width 0.6) (layer "F.Cu") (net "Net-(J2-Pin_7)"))
 (segment (start 203.762696 81.478549) (end 201.978549 81.478549) (width 0.6) (layer "F.Cu") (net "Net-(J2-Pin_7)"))
 (segment (start 203.892073 81.607927) (end 203.762696 81.478549) (width 0.6) (layer "F.Cu") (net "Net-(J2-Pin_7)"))
 (segment (start 200.484172 82.972926) (end 201.978549 81.478549) (width 0.6) (layer "F.Cu") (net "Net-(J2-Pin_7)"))
 (segment (start 203.892073 81.607927) (end 204.135 81.365) (width 0.6) (layer "F.Cu") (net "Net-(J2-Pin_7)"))
 (segment (start 204.135 81.365) (end 204.135 78.4125) (width 0.6) (layer "F.Cu") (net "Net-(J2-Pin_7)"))
 (segment (start 206.531 87.331) (end 206.531 84.246853) (width 0.6) (layer "F.Cu") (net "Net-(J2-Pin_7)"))
 (segment (start 194.527074 82.972926) (end 188.5 89) (width 0.6) (layer "F.Cu") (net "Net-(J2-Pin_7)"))
 (segment (start 206.531 84.246853) (end 203.892073 81.607927) (width 0.6) (layer "F.Cu") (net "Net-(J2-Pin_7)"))
 (segment (start 200.002902 79) (end 201.028902 80.026) (width 0.6) (layer "F.Cu") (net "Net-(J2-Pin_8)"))
 (segment (start 187 78.5) (end 187.5 79) (width 0.6) (layer "F.Cu") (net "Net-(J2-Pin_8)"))
 (segment (start 214.151 84.978902) (end 205.971098 76.799) (width 0.6) (layer "F.Cu") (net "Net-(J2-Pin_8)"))
 (segment (start 214.151 89.109) (end 214.151 84.978902) (width 0.6) (layer "F.Cu") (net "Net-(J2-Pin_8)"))
 (segment (start 187.5 79) (end 200.002902 79) (width 0.6) (layer "F.Cu") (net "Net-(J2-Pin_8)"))
 (segment (start 202.865 79.322098) (end 202.865 78.4125) (width 0.6) (layer "F.Cu") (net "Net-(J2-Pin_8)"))
 (segment (start 203.568902 76.799) (end 202.865 77.502902) (width 0.6) (layer "F.Cu") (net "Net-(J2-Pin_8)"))
 (segment (start 202.865 77.502902) (end 202.865 78.4125) (width 0.6) (layer "F.Cu") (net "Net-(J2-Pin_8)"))
 (segment (start 201.028902 80.026) (end 202.161098 80.026) (width 0.6) (layer "F.Cu") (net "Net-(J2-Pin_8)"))
 (segment (start 205.971098 76.799) (end 203.568902 76.799) (width 0.6) (layer "F.Cu") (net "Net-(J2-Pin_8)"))
 (segment (start 212.5 90.76) (end 214.151 89.109) (width 0.6) (layer "F.Cu") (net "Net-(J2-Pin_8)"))
 (segment (start 202.161098 80.026) (end 202.865 79.322098) (width 0.6) (layer "F.Cu") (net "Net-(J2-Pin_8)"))
 (segment (start 209.154 97.574) (end 204.1845 97.574) (width 0.6) (layer "F.Cu") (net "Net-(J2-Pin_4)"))
 (segment (start 201.595 94.9845) (end 201.595 85.5875) (width 0.6) (layer "F.Cu") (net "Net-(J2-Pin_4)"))
 (segment (start 204.1845 97.574) (end 201.595 94.9845) (width 0.6) (layer "F.Cu") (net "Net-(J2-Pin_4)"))
 (segment (start 212.5 100.92) (end 209.154 97.574) (width 0.6) (layer "F.Cu") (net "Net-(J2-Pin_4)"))
 (segment (start 210.195 96.075) (end 205.2875 96.075) (width 0.6) (layer "F.Cu") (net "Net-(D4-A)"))
 (segment (start 212.5 98.38) (end 210.195 96.075) (width 0.6) (layer "F.Cu") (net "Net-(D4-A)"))
 (segment (start 202.865 93.6525) (end 202.865 85.5875) (width 0.6) (layer "F.Cu") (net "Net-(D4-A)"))
 (segment (start 205.2875 96.075) (end 202.865 93.6525) (width 0.6) (layer "F.Cu") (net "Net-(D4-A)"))
 (segment (start 204.5 93) (end 204.135 92.635) (width 0.6) (layer "F.Cu") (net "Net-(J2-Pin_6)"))
 (segment (start 204.135 92.635) (end 204.135 85.5875) (width 0.6) (layer "F.Cu") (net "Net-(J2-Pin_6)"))
 (segment (start 212.5 95.84) (end 209.66 93) (width 0.6) (layer "F.Cu") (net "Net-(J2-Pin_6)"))
 (segment (start 209.66 93) (end 204.5 93) (width 0.6) (layer "F.Cu") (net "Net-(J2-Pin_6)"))
 (segment (start 188.5 97.5) (end 188.5 96.502902) (width 0.6) (layer "F.Cu") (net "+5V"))
 (segment (start 185.5 106.5) (end 186 106) (width 0.6) (layer "F.Cu") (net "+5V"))
 (segment (start 189.75 113) (end 185.5 108.75) (width 0.6) (layer "F.Cu") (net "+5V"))
 (segment (start 186 106) (end 191.4625 106) (width 0.6) (layer "F.Cu") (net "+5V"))
 (segment (start 196.7125 112.425) (end 208.615 112.425) (width 0.6) (layer "F.Cu") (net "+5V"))
 (segment (start 208.615 112.425) (end 212.5 108.54) (width 0.6) (layer "F.Cu") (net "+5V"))
 (segment (start 205.405 84.677902) (end 205.405 85.5875) (width 0.6) (layer "F.Cu") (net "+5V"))
 (segment (start 204.701098 83.974) (end 205.405 84.677902) (width 0.6) (layer "F.Cu") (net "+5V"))
 (segment (start 191.4625 106) (end 191.9625 105.5) (width 0.6) (layer "F.Cu") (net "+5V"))
 (segment (start 188.5 96.502902) (end 201.028902 83.974) (width 0.6) (layer "F.Cu") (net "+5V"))
 (segment (start 185.5 108.75) (end 185.5 106.5) (width 0.6) (layer "F.Cu") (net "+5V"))
 (segment (start 201.028902 83.974) (end 204.701098 83.974) (width 0.6) (layer "F.Cu") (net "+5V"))
 (segment (start 196.1375 113) (end 196.7125 112.425) (width 0.6) (layer "F.Cu") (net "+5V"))
 (segment (start 191.9625 105.5) (end 191.9625 104.9625) (width 0.6) (layer "F.Cu") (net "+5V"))
 (segment (start 191.9625 104.9625) (end 188.5 101.5) (width 0.6) (layer "F.Cu") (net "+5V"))
 (segment (start 188.5 101.5) (end 188.5 97.5) (width 0.6) (layer "F.Cu") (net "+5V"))
 (segment (start 189.75 113) (end 196.1375 113) (width 0.6) (layer "F.Cu") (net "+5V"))
 (segment (start 196.7125 109.625) (end 203.375 109.625) (width 0.6) (layer "F.Cu") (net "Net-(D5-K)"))
 (segment (start 203.5 109.5) (end 203.5 108) (width 0.6) (layer "F.Cu") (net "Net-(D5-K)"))
 (segment (start 203.375 109.625) (end 203.5 109.5) (width 0.6) (layer "F.Cu") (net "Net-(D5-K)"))
 (segment (start 185.75 113.5) (end 186.25 113) (width 0.6) (layer "F.Cu") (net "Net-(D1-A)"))
 (segment (start 177 113.5) (end 185.75 113.5) (width 0.6) (layer "F.Cu") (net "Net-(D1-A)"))
 (segment (start 186.5 102.85) (end 186.5 103) (width 0.6) (layer "F.Cu") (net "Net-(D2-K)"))
 (segment (start 188.5 91) (end 187.5 91) (width 0.6) (layer "F.Cu") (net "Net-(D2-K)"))
 (segment (start 186.5 103) (end 184 105.5) (width 0.6) (layer "F.Cu") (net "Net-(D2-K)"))
 (segment (start 186.5 102.85) (end 186.5 97.5) (width 0.6) (layer "F.Cu") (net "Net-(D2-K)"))
 (segment (start 188 104.35) (end 186.5 102.85) (width 0.6) (layer "F.Cu") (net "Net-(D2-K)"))
 (segment (start 186.5 97.5) (end 186.5 92) (width 0.6) (layer "F.Cu") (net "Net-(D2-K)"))
 (segment (start 184 111) (end 177.5 111) (width 0.6) (layer "F.Cu") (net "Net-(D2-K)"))
 (segment (start 187.5 91) (end 186.5 92) (width 0.6) (layer "F.Cu") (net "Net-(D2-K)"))
 (segment (start 184 105.5) (end 184 111) (width 0.6) (layer "F.Cu") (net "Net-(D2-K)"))
 (segment (start 200 102) (end 202.1625 102) (width 0.6) (layer "F.Cu") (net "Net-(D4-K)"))
 (segment (start 202.1625 102) (end 205.2875 98.875) (width 0.6) (layer "F.Cu") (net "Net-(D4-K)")))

